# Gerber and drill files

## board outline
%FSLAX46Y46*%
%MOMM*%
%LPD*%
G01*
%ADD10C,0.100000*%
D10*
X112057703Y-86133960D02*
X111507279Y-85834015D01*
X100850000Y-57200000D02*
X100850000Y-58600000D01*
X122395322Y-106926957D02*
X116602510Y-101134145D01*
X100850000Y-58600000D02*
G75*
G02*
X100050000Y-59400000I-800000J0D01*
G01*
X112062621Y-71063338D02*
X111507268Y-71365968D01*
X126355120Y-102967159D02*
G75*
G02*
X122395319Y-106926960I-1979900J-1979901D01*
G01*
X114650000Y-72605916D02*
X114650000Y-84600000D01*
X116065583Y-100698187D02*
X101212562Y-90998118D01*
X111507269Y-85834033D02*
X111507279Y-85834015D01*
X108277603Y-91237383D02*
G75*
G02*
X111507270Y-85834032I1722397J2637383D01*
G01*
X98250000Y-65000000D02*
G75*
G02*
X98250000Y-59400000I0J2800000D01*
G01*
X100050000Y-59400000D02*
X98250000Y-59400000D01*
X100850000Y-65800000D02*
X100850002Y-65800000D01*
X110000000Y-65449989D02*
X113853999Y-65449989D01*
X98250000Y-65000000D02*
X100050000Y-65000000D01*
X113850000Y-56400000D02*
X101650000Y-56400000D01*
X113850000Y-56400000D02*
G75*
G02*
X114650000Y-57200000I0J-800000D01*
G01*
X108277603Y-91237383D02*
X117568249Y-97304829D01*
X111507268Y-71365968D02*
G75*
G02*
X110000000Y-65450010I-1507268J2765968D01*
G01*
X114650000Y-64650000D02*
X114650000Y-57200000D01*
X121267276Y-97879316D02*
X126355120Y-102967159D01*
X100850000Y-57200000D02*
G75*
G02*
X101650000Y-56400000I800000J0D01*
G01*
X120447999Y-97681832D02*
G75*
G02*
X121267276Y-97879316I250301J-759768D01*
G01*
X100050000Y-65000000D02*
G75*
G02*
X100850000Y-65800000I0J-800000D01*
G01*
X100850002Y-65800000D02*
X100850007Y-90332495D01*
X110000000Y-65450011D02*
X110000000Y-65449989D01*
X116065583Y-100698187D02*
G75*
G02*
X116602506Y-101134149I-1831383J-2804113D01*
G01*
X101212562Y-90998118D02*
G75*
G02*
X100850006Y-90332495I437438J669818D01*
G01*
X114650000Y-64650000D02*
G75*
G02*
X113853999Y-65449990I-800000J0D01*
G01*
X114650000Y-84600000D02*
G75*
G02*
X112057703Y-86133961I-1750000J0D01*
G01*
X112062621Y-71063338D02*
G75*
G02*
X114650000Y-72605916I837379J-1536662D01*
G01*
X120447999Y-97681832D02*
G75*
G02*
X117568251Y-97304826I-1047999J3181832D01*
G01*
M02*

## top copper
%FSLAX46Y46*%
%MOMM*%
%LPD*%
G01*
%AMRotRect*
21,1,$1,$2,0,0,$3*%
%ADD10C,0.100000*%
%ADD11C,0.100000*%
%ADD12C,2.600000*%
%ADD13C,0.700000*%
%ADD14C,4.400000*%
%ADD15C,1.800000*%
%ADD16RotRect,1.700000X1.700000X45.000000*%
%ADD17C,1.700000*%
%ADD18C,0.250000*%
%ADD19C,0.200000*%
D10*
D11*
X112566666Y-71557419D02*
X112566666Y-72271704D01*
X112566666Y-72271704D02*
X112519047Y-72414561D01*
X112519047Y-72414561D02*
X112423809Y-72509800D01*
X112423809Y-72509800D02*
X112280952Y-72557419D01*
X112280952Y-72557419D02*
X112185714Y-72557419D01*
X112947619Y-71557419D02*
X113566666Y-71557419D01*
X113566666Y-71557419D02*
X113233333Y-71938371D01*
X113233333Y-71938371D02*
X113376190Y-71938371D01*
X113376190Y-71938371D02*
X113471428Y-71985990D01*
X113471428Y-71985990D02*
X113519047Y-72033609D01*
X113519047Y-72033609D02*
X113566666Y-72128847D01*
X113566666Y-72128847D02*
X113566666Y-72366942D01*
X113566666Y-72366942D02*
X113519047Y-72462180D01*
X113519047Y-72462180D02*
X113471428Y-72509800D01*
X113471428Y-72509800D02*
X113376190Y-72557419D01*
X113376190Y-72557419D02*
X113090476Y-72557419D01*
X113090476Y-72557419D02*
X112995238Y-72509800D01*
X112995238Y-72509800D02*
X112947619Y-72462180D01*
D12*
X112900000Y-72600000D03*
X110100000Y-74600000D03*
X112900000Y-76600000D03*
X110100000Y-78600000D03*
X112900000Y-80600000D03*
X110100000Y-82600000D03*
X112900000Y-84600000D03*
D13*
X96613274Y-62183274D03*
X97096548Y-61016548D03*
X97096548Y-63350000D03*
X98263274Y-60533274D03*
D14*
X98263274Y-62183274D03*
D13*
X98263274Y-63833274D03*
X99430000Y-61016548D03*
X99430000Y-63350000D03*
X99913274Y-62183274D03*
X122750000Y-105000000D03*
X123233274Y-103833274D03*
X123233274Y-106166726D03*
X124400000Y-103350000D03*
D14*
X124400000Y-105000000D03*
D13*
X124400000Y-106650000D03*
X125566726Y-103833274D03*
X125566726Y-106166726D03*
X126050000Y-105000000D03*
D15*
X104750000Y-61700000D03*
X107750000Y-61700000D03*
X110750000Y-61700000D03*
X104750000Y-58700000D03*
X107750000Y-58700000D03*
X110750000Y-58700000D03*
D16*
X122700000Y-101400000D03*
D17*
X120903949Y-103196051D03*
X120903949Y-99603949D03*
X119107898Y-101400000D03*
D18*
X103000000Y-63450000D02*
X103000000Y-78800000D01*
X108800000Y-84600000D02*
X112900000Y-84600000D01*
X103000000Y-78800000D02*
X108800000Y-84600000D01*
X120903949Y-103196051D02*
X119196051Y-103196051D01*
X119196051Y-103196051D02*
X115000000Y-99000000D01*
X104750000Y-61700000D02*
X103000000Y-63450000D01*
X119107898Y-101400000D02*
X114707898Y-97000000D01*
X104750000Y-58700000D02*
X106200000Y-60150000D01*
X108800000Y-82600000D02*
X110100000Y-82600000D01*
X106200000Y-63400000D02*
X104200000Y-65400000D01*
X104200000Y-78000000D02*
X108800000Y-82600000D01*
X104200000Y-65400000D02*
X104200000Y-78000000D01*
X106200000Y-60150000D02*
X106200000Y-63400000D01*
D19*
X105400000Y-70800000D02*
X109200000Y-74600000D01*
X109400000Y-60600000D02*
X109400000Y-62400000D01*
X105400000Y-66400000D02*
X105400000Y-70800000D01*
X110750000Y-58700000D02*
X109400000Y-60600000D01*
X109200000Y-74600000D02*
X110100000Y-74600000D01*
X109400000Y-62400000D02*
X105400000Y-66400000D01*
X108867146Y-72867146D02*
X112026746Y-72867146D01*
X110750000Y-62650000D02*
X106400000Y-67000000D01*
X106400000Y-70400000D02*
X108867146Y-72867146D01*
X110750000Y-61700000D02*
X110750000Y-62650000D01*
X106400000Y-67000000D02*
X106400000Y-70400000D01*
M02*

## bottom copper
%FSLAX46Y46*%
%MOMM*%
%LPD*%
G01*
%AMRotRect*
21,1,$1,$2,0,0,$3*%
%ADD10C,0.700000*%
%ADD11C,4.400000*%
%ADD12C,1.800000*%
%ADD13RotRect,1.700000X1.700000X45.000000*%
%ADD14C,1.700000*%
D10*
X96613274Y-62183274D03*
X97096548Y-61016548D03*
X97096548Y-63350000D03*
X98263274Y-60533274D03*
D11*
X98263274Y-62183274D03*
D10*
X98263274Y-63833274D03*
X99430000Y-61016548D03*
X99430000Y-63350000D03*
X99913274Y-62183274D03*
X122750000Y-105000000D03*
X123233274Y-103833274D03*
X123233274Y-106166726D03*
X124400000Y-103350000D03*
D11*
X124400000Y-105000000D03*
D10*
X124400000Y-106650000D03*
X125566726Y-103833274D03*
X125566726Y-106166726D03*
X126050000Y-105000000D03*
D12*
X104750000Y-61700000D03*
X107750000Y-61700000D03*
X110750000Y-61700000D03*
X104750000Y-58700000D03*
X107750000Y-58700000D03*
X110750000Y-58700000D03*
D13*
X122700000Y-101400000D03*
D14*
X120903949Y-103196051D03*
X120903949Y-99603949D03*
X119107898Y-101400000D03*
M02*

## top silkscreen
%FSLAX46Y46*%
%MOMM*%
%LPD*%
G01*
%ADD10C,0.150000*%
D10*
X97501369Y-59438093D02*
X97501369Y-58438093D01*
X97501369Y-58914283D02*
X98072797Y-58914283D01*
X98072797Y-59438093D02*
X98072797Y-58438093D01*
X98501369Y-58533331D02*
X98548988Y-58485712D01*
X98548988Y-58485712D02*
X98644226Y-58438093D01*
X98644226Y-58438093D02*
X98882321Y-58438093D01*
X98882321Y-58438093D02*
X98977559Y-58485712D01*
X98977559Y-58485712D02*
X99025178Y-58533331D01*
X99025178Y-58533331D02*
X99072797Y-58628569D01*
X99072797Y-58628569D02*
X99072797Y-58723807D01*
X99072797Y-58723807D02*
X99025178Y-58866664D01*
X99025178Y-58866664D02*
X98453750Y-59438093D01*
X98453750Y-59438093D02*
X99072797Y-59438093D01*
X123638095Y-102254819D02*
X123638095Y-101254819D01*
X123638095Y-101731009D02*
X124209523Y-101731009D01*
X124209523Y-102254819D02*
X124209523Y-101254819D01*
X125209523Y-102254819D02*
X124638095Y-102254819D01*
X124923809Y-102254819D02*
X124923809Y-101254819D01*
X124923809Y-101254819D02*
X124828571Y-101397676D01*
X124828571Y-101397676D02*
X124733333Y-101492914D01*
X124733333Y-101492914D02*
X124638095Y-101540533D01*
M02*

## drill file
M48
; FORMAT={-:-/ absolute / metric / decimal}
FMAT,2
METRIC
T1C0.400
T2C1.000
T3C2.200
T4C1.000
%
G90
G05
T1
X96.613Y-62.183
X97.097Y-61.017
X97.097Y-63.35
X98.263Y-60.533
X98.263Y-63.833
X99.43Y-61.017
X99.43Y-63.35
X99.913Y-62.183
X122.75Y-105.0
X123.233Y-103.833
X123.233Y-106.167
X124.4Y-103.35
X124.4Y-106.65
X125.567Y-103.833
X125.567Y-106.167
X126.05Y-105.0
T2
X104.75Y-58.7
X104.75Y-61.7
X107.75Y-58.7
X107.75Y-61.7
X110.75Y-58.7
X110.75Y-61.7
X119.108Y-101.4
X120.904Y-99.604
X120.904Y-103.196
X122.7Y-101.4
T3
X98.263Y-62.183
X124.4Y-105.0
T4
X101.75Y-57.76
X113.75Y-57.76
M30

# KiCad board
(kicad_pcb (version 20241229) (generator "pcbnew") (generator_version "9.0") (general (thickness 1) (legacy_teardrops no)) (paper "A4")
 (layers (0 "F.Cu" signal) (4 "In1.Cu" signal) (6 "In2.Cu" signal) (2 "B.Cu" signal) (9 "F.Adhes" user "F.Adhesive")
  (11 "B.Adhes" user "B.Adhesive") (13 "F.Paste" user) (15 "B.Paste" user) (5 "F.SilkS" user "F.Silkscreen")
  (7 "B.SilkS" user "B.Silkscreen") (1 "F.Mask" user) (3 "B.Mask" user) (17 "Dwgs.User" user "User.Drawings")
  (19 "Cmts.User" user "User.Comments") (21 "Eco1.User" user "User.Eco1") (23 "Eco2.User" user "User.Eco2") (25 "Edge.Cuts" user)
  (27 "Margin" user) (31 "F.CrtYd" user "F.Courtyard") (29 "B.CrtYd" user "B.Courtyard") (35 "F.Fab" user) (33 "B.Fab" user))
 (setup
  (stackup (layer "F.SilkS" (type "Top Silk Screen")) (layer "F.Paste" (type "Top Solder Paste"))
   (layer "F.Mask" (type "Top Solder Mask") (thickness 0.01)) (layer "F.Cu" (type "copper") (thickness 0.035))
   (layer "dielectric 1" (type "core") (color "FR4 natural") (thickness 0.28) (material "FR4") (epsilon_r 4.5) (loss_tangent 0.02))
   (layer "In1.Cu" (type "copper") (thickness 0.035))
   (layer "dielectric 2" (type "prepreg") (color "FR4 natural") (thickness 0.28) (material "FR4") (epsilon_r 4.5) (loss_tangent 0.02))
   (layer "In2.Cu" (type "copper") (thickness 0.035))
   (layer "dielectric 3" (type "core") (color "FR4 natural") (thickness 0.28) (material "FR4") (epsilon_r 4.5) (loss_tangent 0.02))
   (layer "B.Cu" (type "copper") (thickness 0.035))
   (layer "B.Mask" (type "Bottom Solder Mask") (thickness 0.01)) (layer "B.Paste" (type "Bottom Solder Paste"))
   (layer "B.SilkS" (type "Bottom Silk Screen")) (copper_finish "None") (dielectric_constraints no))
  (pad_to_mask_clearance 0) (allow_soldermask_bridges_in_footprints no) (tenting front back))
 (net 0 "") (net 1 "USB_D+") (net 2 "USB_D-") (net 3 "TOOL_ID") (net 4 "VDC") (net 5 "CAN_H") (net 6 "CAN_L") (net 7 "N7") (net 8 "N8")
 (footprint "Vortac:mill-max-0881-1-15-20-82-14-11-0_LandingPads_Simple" (layer "F.Cu") (at 112.9 72.6)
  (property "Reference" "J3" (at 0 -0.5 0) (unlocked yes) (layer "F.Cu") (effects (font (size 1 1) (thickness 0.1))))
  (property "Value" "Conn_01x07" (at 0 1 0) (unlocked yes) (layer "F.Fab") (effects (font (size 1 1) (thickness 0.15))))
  (pad "1" smd circle (at 0 0) (size 2.6 2.6) (layers "F.Cu" "F.Mask") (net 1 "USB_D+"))
  (pad "2" smd circle (at -2.8 2) (size 2.6 2.6) (layers "F.Cu" "F.Mask") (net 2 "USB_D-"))
  (pad "3" smd circle (at 0 4) (size 2.6 2.6) (layers "F.Cu" "F.Mask") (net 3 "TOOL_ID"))
  (pad "4" smd circle (at -2.8 6) (size 2.6 2.6) (layers "F.Cu" "F.Mask") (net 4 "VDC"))
  (pad "5" smd circle (at 0 8) (size 2.6 2.6) (layers "F.Cu" "F.Mask") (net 3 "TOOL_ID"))
  (pad "6" smd circle (at -2.8 10) (size 2.6 2.6) (layers "F.Cu" "F.Mask") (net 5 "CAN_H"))
  (pad "7" smd circle (at 0 12) (size 2.6 2.6) (layers "F.Cu" "F.Mask") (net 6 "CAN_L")))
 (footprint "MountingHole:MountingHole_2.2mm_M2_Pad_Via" (layer "F.Cu") (at 98.263274 62.183274)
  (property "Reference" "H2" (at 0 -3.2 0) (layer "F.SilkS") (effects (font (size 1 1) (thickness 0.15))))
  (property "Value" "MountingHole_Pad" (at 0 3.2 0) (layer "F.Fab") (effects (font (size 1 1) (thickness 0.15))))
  (pad "1" thru_hole circle (at -1.65 0) (size 0.7 0.7) (drill 0.4) (layers "*.Cu" "*.Mask") (remove_unused_layers no) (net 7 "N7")
   (zone_connect 2))
  (pad "1" thru_hole circle (at -1.166726 -1.166726) (size 0.7 0.7) (drill 0.4) (layers "*.Cu" "*.Mask") (remove_unused_layers no)
   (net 7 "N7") (zone_connect 2))
  (pad "1" thru_hole circle (at -1.166726 1.166726) (size 0.7 0.7) (drill 0.4) (layers "*.Cu" "*.Mask") (remove_unused_layers no)
   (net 7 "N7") (zone_connect 2))
  (pad "1" thru_hole circle (at 0 -1.65) (size 0.7 0.7) (drill 0.4) (layers "*.Cu" "*.Mask") (remove_unused_layers no) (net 7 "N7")
   (zone_connect 2))
  (pad "1" thru_hole circle (at 0 0) (size 4.4 4.4) (drill 2.2) (layers "*.Cu" "*.Mask") (remove_unused_layers no) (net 7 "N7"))
  (pad "1" thru_hole circle (at 0 1.65) (size 0.7 0.7) (drill 0.4) (layers "*.Cu" "*.Mask") (remove_unused_layers no) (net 7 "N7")
   (zone_connect 2))
  (pad "1" thru_hole circle (at 1.166726 -1.166726) (size 0.7 0.7) (drill 0.4) (layers "*.Cu" "*.Mask") (remove_unused_layers no)
   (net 7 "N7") (zone_connect 2))
  (pad "1" thru_hole circle (at 1.166726 1.166726) (size 0.7 0.7) (drill 0.4) (layers "*.Cu" "*.Mask") (remove_unused_layers no)
   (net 7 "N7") (zone_connect 2))
  (pad "1" thru_hole circle (at 1.65 0) (size 0.7 0.7) (drill 0.4) (layers "*.Cu" "*.Mask") (remove_unused_layers no) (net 7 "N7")
   (zone_connect 2)))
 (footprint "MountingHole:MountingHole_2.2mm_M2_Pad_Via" (layer "F.Cu") (at 124.4 105)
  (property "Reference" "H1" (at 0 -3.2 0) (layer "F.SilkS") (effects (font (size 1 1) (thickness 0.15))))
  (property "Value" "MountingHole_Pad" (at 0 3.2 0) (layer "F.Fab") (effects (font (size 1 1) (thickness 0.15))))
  (pad "1" thru_hole circle (at -1.65 0) (size 0.7 0.7) (drill 0.4) (layers "*.Cu" "*.Mask") (remove_unused_layers no) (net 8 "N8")
   (zone_connect 2))
  (pad "1" thru_hole circle (at -1.166726 -1.166726) (size 0.7 0.7) (drill 0.4) (layers "*.Cu" "*.Mask") (remove_unused_layers no)
   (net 8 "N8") (zone_connect 2))
  (pad "1" thru_hole circle (at -1.166726 1.166726) (size 0.7 0.7) (drill 0.4) (layers "*.Cu" "*.Mask") (remove_unused_layers no)
   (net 8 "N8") (zone_connect 2))
  (pad "1" thru_hole circle (at 0 -1.65) (size 0.7 0.7) (drill 0.4) (layers "*.Cu" "*.Mask") (remove_unused_layers no) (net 8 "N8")
   (zone_connect 2))
  (pad "1" thru_hole circle (at 0 0) (size 4.4 4.4) (drill 2.2) (layers "*.Cu" "*.Mask") (remove_unused_layers no) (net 8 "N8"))
  (pad "1" thru_hole circle (at 0 1.65) (size 0.7 0.7) (drill 0.4) (layers "*.Cu" "*.Mask") (remove_unused_layers no) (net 8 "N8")
   (zone_connect 2))
  (pad "1" thru_hole circle (at 1.166726 -1.166726) (size 0.7 0.7) (drill 0.4) (layers "*.Cu" "*.Mask") (remove_unused_layers no)
   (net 8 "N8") (zone_connect 2))
  (pad "1" thru_hole circle (at 1.166726 1.166726) (size 0.7 0.7) (drill 0.4) (layers "*.Cu" "*.Mask") (remove_unused_layers no)
   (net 8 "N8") (zone_connect 2))
  (pad "1" thru_hole circle (at 1.65 0) (size 0.7 0.7) (drill 0.4) (layers "*.Cu" "*.Mask") (remove_unused_layers no) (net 8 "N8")
   (zone_connect 2)))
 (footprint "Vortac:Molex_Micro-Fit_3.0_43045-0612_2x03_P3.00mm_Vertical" (layer "B.Cu") (at 104.75 61.7)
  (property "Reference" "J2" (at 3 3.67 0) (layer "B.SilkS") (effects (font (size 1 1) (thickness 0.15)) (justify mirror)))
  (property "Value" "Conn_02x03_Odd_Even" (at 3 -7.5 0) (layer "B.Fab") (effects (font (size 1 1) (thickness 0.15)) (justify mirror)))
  (pad "" np_thru_hole circle (at -3 -3.94) (size 1 1) (drill 1) (layers "*.Cu" "*.Mask"))
  (pad "" np_thru_hole circle (at 9 -3.94) (size 1 1) (drill 1) (layers "*.Cu" "*.Mask"))
  (pad "1" thru_hole circle (at 0 0) (size 1.8 1.8) (drill 1) (layers "*.Cu" "*.Mask") (remove_unused_layers no) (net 6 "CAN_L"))
  (pad "2" thru_hole circle (at 3 0) (size 1.8 1.8) (drill 1) (layers "*.Cu" "*.Mask") (remove_unused_layers no) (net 3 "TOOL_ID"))
  (pad "3" thru_hole circle (at 6 0) (size 1.8 1.8) (drill 1) (layers "*.Cu" "*.Mask") (remove_unused_layers no) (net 1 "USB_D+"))
  (pad "4" thru_hole circle (at 0 -3) (size 1.8 1.8) (drill 1) (layers "*.Cu" "*.Mask") (remove_unused_layers no) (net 5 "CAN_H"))
  (pad "5" thru_hole circle (at 3 -3) (size 1.8 1.8) (drill 1) (layers "*.Cu" "*.Mask") (remove_unused_layers no) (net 4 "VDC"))
  (pad "6" thru_hole circle (at 6 -3) (size 1.8 1.8) (drill 1) (layers "*.Cu" "*.Mask") (remove_unused_layers no) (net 2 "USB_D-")))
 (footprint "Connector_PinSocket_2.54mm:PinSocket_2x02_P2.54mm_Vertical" (layer "B.Cu") (at 122.7 101.4 45)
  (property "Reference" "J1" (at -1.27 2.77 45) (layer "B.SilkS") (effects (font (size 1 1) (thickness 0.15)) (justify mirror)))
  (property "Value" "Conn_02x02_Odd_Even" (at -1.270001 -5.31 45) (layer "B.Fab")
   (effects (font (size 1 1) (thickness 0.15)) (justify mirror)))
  (pad "1" thru_hole rect (at 0 0 45) (size 1.7 1.7) (drill 1) (layers "*.Cu" "*.Mask") (remove_unused_layers no) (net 3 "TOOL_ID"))
  (pad "2" thru_hole circle (at -2.54 0 45) (size 1.7 1.7) (drill 1) (layers "*.Cu" "*.Mask") (remove_unused_layers no) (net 6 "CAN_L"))
  (pad "3" thru_hole circle (at 0 -2.54 45) (size 1.7 1.7) (drill 1) (layers "*.Cu" "*.Mask") (remove_unused_layers no) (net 4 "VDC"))
  (pad "4" thru_hole circle (at -2.54 -2.54 45) (size 1.7 1.7) (drill 1) (layers "*.Cu" "*.Mask") (remove_unused_layers no) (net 5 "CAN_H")))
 (gr_line (start 112.057703 86.13396) (end 111.507279 85.834015) (stroke (width 0.1) (type default)) (layer "Edge.Cuts"))
 (gr_line (start 100.85 57.2) (end 100.85 58.6) (stroke (width 0.1) (type default)) (layer "Edge.Cuts"))
 (gr_line (start 122.395322 106.926957) (end 116.60251 101.134145) (stroke (width 0.1) (type default)) (layer "Edge.Cuts"))
 (gr_arc (start 100.85 58.6) (mid 100.615685 59.165685) (end 100.05 59.4) (stroke (width 0.1) (type default)) (layer "Edge.Cuts"))
 (gr_line (start 112.062621 71.063338) (end 111.507268 71.365968) (stroke (width 0.1) (type default)) (layer "Edge.Cuts"))
 (gr_arc (start 126.35512 102.967159) (mid 126.355122 106.926959) (end 122.395322 106.926957) (stroke (width 0.1) (type default))
  (layer "Edge.Cuts"))
 (gr_line (start 114.65 72.605916) (end 114.65 84.6) (stroke (width 0.1) (type default)) (layer "Edge.Cuts"))
 (gr_line (start 116.065583 100.698187) (end 101.212562 90.998118) (stroke (width 0.1) (type default)) (layer "Edge.Cuts"))
 (gr_line (start 111.507269 85.834033) (end 111.507279 85.834015) (stroke (width 0.1) (type default)) (layer "Edge.Cuts"))
 (gr_arc (start 108.277603 91.237383) (mid 107.296184 86.983887) (end 111.507269 85.834033) (stroke (width 0.1) (type default))
  (layer "Edge.Cuts"))
 (gr_arc (start 98.25 65) (mid 95.45 62.2) (end 98.25 59.4) (stroke (width 0.1) (type default)) (layer "Edge.Cuts"))
 (gr_line (start 100.05 59.4) (end 98.25 59.4) (stroke (width 0.1) (type default)) (layer "Edge.Cuts"))
 (gr_line (start 100.85 65.8) (end 100.850002 65.8) (stroke (width 0.1) (type default)) (layer "Edge.Cuts"))
 (gr_line (start 110 65.449989) (end 113.853999 65.449989) (stroke (width 0.1) (type default)) (layer "Edge.Cuts"))
 (gr_line (start 98.25 65) (end 100.05 65) (stroke (width 0.1) (type default)) (layer "Edge.Cuts"))
 (gr_line (start 113.85 56.4) (end 101.65 56.4) (stroke (width 0.1) (type default)) (layer "Edge.Cuts"))
 (gr_arc (start 113.85 56.4) (mid 114.415685 56.634315) (end 114.65 57.2) (stroke (width 0.1) (type default)) (layer "Edge.Cuts"))
 (gr_line (start 108.277603 91.237383) (end 117.568249 97.304829) (stroke (width 0.1) (type default)) (layer "Edge.Cuts"))
 (gr_arc (start 111.507268 71.365968) (mid 106.947526 69.377713) (end 110 65.450011) (stroke (width 0.1) (type default)) (layer "Edge.Cuts"))
 (gr_line (start 114.65 64.65) (end 114.65 57.2) (stroke (width 0.1) (type default)) (layer "Edge.Cuts"))
 (gr_line (start 121.267276 97.879316) (end 126.35512 102.967159) (stroke (width 0.1) (type default)) (layer "Edge.Cuts"))
 (gr_arc (start 100.85 57.2) (mid 101.084315 56.634315) (end 101.65 56.4) (stroke (width 0.1) (type default)) (layer "Edge.Cuts"))
 (gr_arc (start 120.447999 97.681832) (mid 120.88347 97.663393) (end 121.267276 97.879316) (stroke (width 0.1) (type default))
  (layer "Edge.Cuts"))
 (gr_arc (start 100.05 65) (mid 100.615686 65.234315) (end 100.85 65.8) (stroke (width 0.1) (type default)) (layer "Edge.Cuts"))
 (gr_line (start 100.850002 65.8) (end 100.850007 90.332495) (stroke (width 0.1) (type default)) (layer "Edge.Cuts"))
 (gr_line (start 110 65.450011) (end 110 65.449989) (stroke (width 0.1) (type default)) (layer "Edge.Cuts"))
 (gr_arc (start 116.065583 100.698187) (mid 116.345275 100.902224) (end 116.60251 101.134145) (stroke (width 0.1) (type default))
  (layer "Edge.Cuts"))
 (gr_arc (start 101.212562 90.998118) (mid 100.946457 90.709136) (end 100.850007 90.332495) (stroke (width 0.1) (type default))
  (layer "Edge.Cuts"))
 (gr_arc (start 114.65 64.65) (mid 114.415689 65.215682) (end 113.853999 65.449989) (stroke (width 0.1) (type default)) (layer "Edge.Cuts"))
 (gr_arc (start 114.65 84.6) (mid 113.793617 86.104642) (end 112.057703 86.13396) (stroke (width 0.1) (type default)) (layer "Edge.Cuts"))
 (gr_arc (start 112.062621 71.063338) (mid 113.793618 71.095347) (end 114.65 72.605916) (stroke (width 0.1) (type default))
  (layer "Edge.Cuts"))
 (gr_arc (start 120.447999 97.681832) (mid 118.965138 97.821634) (end 117.568249 97.304829) (stroke (width 0.1) (type default))
  (layer "Edge.Cuts"))
 (segment (start 103 63.45) (end 103 78.8) (width 0.25) (layer "F.Cu") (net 6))
 (segment (start 108.8 84.6) (end 112.9 84.6) (width 0.25) (layer "F.Cu") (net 6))
 (segment (start 103 78.8) (end 108.8 84.6) (width 0.25) (layer "F.Cu") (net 6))
 (segment (start 120.903949 103.196051) (end 119.196051 103.196051) (width 0.25) (layer "F.Cu") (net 6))
 (segment (start 119.196051 103.196051) (end 115 99) (width 0.25) (layer "F.Cu") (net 6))
 (segment (start 104.75 61.7) (end 103 63.45) (width 0.25) (layer "F.Cu") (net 6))
 (segment (start 119.107898 101.4) (end 114.707898 97) (width 0.25) (layer "F.Cu") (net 5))
 (segment (start 104.75 58.7) (end 106.2 60.15) (width 0.25) (layer "F.Cu") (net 5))
 (segment (start 108.8 82.6) (end 110.1 82.6) (width 0.25) (layer "F.Cu") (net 5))
 (segment (start 106.2 63.4) (end 104.2 65.4) (width 0.25) (layer "F.Cu") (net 5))
 (segment (start 104.2 78) (end 108.8 82.6) (width 0.25) (layer "F.Cu") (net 5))
 (segment (start 104.2 65.4) (end 104.2 78) (width 0.25) (layer "F.Cu") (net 5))
 (segment (start 106.2 60.15) (end 106.2 63.4) (width 0.25) (layer "F.Cu") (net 5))
 (segment (start 105.4 70.8) (end 109.2 74.6) (width 0.2) (layer "F.Cu") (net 2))
 (segment (start 109.4 60.6) (end 109.4 62.4) (width 0.2) (layer "F.Cu") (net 2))
 (segment (start 105.4 66.4) (end 105.4 70.8) (width 0.2) (layer "F.Cu") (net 2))
 (segment (start 110.75 58.7) (end 109.4 60.6) (width 0.2) (layer "F.Cu") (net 2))
 (segment (start 109.2 74.6) (end 110.1 74.6) (width 0.2) (layer "F.Cu") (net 2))
 (segment (start 109.4 62.4) (end 105.4 66.4) (width 0.2) (layer "F.Cu") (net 2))
 (segment (start 108.867146 72.867146) (end 112.026746 72.867146) (width 0.2) (layer "F.Cu") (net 1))
 (segment (start 110.75 62.65) (end 106.4 67) (width 0.2) (layer "F.Cu") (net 1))
 (segment (start 106.4 70.4) (end 108.867146 72.867146) (width 0.2) (layer "F.Cu") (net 1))
 (segment (start 110.75 61.7) (end 110.75 62.65) (width 0.2) (layer "F.Cu") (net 1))
 (segment (start 106.4 67) (end 106.4 70.4) (width 0.2) (layer "F.Cu") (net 1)))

